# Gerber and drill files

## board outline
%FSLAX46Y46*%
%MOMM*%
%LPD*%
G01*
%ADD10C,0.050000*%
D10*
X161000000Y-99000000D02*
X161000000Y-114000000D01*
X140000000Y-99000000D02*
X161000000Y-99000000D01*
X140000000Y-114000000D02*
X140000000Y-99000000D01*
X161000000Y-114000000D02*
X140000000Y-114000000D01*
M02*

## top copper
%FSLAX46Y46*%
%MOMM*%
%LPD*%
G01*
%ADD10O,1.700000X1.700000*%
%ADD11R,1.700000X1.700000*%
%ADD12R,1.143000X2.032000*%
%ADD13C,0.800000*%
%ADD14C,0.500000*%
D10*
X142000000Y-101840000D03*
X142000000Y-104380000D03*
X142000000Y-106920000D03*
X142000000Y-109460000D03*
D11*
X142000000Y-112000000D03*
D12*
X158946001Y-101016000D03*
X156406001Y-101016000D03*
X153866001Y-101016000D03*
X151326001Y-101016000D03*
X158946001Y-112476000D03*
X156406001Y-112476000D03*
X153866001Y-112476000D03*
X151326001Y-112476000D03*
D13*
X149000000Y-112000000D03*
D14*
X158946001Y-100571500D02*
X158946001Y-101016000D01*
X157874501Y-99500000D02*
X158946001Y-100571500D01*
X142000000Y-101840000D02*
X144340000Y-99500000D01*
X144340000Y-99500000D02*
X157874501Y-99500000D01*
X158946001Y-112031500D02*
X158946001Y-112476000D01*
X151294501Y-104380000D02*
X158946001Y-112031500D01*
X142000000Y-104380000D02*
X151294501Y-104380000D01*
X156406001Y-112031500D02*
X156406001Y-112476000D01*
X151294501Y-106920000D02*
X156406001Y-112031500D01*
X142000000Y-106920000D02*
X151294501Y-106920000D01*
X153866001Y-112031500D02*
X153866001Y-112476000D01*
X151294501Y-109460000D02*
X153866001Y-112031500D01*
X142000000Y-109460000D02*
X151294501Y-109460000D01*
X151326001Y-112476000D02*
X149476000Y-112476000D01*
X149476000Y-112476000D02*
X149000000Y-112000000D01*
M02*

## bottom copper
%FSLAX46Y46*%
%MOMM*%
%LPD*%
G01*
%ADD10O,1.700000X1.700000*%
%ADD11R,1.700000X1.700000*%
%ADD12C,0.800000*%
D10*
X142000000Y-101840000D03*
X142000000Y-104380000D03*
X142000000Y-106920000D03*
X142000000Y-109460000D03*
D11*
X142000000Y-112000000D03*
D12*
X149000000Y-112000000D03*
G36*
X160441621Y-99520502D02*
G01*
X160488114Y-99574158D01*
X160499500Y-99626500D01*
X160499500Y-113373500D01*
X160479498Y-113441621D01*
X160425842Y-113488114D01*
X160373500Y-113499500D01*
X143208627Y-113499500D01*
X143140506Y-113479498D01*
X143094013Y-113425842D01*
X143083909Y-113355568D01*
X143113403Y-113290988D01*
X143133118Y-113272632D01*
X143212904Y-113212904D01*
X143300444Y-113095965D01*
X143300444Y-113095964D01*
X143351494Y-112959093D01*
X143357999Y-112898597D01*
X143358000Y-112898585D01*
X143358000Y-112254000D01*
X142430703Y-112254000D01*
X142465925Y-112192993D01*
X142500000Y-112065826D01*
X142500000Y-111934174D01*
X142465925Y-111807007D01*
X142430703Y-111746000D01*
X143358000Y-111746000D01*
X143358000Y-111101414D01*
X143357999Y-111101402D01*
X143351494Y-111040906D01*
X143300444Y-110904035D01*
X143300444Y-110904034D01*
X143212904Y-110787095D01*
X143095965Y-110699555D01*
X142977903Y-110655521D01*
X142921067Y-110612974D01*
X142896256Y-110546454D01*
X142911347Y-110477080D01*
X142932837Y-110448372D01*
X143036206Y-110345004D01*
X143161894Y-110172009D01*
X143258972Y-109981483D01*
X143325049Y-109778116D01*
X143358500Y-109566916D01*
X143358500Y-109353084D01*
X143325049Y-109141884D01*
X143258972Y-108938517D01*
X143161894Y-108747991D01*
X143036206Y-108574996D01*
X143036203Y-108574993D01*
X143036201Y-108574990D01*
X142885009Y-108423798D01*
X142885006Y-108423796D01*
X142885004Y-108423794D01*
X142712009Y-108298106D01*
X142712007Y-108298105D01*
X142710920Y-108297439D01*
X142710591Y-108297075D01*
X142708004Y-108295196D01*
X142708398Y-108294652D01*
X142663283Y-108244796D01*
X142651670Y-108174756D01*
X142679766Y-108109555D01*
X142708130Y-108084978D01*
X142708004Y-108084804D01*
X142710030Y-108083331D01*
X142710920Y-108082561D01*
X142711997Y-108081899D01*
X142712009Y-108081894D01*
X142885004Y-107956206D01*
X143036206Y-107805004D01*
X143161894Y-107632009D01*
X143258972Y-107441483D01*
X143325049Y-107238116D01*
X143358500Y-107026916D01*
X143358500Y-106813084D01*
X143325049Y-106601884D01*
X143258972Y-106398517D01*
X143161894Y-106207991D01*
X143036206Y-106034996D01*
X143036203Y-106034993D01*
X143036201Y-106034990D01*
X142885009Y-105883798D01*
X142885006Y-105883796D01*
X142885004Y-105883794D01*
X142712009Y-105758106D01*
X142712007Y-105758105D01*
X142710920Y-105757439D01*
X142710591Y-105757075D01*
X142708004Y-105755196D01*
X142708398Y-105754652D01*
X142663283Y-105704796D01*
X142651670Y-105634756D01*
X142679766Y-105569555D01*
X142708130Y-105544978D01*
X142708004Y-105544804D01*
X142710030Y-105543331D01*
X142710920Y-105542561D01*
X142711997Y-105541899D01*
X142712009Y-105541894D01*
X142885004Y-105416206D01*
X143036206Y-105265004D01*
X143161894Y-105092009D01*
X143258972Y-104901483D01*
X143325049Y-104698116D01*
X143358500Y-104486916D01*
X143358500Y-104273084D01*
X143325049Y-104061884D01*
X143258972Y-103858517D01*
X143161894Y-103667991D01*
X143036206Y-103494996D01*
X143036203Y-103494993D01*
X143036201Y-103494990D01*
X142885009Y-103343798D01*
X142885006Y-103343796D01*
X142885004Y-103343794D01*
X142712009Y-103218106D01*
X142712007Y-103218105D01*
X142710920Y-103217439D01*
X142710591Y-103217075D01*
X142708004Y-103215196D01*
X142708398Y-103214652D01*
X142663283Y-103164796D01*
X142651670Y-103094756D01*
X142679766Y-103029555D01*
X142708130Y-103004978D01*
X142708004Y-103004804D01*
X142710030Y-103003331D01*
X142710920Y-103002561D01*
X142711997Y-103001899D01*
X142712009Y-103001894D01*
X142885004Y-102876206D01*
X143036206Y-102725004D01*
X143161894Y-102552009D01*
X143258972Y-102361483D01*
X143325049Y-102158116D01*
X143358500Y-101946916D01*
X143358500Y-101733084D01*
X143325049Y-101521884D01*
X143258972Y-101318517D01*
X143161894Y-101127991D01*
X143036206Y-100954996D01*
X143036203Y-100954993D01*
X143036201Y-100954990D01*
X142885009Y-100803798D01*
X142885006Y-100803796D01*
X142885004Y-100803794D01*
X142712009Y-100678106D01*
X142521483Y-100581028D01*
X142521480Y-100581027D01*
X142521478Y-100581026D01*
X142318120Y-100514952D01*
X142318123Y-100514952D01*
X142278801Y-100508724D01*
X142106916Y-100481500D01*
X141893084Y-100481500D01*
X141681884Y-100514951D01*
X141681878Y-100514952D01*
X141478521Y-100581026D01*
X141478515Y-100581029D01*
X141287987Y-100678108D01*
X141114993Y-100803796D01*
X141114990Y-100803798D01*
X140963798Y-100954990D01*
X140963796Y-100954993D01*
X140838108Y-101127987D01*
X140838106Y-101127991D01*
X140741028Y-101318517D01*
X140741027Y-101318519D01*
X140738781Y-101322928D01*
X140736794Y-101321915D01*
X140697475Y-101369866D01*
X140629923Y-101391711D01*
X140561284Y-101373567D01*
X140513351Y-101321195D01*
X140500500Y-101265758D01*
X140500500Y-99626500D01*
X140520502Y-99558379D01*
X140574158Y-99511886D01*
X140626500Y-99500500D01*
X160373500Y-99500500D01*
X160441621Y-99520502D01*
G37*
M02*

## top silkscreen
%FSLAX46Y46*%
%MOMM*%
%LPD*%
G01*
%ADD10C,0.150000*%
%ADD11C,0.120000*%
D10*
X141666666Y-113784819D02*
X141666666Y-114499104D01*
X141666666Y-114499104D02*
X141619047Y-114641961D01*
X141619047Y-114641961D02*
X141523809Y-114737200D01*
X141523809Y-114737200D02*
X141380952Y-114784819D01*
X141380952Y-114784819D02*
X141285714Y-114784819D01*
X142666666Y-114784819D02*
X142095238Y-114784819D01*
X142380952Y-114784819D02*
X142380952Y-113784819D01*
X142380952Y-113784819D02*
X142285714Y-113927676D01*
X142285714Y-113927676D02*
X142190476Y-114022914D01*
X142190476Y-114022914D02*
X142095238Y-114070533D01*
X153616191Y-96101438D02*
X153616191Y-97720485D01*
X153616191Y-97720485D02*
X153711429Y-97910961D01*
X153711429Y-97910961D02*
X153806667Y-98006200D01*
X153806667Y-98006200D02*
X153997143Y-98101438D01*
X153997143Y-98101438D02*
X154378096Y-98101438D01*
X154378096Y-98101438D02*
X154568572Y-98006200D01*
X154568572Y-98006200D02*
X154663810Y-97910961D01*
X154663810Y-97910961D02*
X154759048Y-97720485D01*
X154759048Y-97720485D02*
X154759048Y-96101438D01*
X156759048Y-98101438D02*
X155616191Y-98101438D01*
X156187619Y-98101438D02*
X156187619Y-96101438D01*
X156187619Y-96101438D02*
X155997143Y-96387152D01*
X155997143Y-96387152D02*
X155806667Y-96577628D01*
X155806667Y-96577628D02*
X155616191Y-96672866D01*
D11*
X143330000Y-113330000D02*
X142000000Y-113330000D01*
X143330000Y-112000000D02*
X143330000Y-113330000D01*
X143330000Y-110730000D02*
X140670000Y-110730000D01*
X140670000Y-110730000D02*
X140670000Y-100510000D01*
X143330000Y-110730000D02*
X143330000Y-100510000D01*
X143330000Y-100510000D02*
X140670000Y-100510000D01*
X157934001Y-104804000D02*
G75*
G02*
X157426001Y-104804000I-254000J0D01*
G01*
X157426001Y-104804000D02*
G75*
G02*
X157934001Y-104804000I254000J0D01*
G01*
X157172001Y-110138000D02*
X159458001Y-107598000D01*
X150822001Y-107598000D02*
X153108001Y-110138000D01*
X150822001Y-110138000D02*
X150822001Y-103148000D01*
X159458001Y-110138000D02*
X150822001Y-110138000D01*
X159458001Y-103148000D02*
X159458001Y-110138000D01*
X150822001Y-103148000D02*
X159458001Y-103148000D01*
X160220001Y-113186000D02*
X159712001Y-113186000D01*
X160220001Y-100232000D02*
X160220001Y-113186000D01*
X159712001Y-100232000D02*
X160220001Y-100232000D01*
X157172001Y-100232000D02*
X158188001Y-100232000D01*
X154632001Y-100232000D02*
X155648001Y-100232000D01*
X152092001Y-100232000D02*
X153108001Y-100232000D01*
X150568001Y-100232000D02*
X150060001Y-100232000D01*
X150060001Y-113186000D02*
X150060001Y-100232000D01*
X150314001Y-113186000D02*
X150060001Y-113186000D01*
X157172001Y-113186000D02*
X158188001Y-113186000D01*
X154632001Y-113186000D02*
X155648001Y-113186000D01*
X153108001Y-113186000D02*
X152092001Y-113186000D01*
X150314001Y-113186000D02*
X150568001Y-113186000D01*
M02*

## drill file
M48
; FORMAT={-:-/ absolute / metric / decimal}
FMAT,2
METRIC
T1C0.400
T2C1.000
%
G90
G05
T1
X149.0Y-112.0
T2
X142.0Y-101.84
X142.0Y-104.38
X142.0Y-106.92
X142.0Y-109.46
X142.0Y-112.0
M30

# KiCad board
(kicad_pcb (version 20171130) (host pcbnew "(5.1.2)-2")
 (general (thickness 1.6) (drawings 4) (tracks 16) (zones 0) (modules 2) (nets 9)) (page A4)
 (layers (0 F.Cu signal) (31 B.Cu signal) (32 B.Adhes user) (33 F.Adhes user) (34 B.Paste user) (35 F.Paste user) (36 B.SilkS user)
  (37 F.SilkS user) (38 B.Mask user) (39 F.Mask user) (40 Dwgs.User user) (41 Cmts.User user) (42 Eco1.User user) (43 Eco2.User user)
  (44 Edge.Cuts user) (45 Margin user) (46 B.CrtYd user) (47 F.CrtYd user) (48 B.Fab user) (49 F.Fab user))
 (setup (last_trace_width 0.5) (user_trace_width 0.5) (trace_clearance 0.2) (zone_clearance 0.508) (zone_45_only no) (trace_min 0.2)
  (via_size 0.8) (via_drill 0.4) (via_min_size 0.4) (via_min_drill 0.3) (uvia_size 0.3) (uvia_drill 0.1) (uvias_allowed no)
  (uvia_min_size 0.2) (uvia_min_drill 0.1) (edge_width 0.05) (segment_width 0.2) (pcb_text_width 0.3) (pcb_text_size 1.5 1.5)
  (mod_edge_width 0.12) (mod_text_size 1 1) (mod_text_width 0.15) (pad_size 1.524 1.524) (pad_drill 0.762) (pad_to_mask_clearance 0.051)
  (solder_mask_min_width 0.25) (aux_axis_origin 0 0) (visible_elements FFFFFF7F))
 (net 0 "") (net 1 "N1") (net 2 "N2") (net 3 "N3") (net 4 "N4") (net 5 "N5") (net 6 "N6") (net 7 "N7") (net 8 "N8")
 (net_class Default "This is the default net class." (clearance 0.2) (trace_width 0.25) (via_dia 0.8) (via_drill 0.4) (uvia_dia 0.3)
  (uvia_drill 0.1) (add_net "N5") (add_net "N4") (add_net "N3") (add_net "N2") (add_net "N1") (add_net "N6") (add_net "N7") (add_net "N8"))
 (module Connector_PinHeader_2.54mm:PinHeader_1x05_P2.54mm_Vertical (layer F.Cu) (at 142 112 180)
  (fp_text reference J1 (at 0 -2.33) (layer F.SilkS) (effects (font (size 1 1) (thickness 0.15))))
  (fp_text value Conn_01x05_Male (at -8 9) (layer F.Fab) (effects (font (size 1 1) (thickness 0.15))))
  (fp_line (start -1.33 -1.33) (end 0 -1.33) (layer F.SilkS) (width 0.12))
  (fp_line (start -1.33 0) (end -1.33 -1.33) (layer F.SilkS) (width 0.12))
  (fp_line (start -1.33 1.27) (end 1.33 1.27) (layer F.SilkS) (width 0.12))
  (fp_line (start 1.33 1.27) (end 1.33 11.49) (layer F.SilkS) (width 0.12))
  (fp_line (start -1.33 1.27) (end -1.33 11.49) (layer F.SilkS) (width 0.12))
  (fp_line (start -1.33 11.49) (end 1.33 11.49) (layer F.SilkS) (width 0.12))
  (pad 5 thru_hole oval (at 0 10.16 180) (size 1.7 1.7) (drill 1) (layers *.Cu *.Mask) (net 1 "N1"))
  (pad 4 thru_hole oval (at 0 7.62 180) (size 1.7 1.7) (drill 1) (layers *.Cu *.Mask) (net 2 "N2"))
  (pad 3 thru_hole oval (at 0 5.08 180) (size 1.7 1.7) (drill 1) (layers *.Cu *.Mask) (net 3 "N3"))
  (pad 2 thru_hole oval (at 0 2.54 180) (size 1.7 1.7) (drill 1) (layers *.Cu *.Mask) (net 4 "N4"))
  (pad 1 thru_hole rect (at 0 0 180) (size 1.7 1.7) (drill 1) (layers *.Cu *.Mask) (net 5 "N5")))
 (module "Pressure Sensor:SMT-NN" (layer F.Cu) (at 155.140001 107.598)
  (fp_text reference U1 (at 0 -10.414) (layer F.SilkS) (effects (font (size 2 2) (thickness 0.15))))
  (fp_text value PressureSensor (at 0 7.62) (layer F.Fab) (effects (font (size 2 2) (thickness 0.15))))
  (fp_circle (center 2.54 -2.794) (end 2.54 -3.048) (layer F.SilkS) (width 0.12))
  (fp_line (start 2.032 2.54) (end 4.318 0) (layer F.SilkS) (width 0.12))
  (fp_line (start -4.318 0) (end -2.032 2.54) (layer F.SilkS) (width 0.12))
  (fp_line (start -4.318 2.54) (end -4.318 -4.45) (layer F.SilkS) (width 0.12))
  (fp_line (start 4.318 2.54) (end -4.318 2.54) (layer F.SilkS) (width 0.12))
  (fp_line (start 4.318 -4.45) (end 4.318 2.54) (layer F.SilkS) (width 0.12))
  (fp_line (start -4.318 -4.45) (end 4.318 -4.45) (layer F.SilkS) (width 0.12))
  (fp_line (start 5.08 5.588) (end 4.572 5.588) (layer F.SilkS) (width 0.12))
  (fp_line (start 5.08 -7.366) (end 5.08 5.588) (layer F.SilkS) (width 0.12))
  (fp_line (start 4.572 -7.366) (end 5.08 -7.366) (layer F.SilkS) (width 0.12))
  (fp_line (start 2.032 -7.366) (end 3.048 -7.366) (layer F.SilkS) (width 0.12))
  (fp_line (start -0.508 -7.366) (end 0.508 -7.366) (layer F.SilkS) (width 0.12))
  (fp_line (start -3.048 -7.366) (end -2.032 -7.366) (layer F.SilkS) (width 0.12))
  (fp_line (start -4.572 -7.366) (end -5.08 -7.366) (layer F.SilkS) (width 0.12))
  (fp_line (start -5.08 5.588) (end -5.08 -7.366) (layer F.SilkS) (width 0.12))
  (fp_line (start -4.826 5.588) (end -5.08 5.588) (layer F.SilkS) (width 0.12))
  (fp_line (start 2.032 5.588) (end 3.048 5.588) (layer F.SilkS) (width 0.12))
  (fp_line (start -0.508 5.588) (end 0.508 5.588) (layer F.SilkS) (width 0.12))
  (fp_line (start -2.032 5.588) (end -3.048 5.588) (layer F.SilkS) (width 0.12))
  (fp_line (start -4.826 5.588) (end -4.572 5.588) (layer F.SilkS) (width 0.12))
  (pad 5 smd rect (at 3.806 -6.582) (size 1.143 2.032) (layers F.Cu F.Paste F.Mask) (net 1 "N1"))
  (pad 6 smd rect (at 1.266 -6.582) (size 1.143 2.032) (layers F.Cu F.Paste F.Mask) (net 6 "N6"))
  (pad 7 smd rect (at -1.274 -6.582) (size 1.143 2.032) (layers F.Cu F.Paste F.Mask) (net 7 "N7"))
  (pad 8 smd rect (at -3.814 -6.582) (size 1.143 2.032) (layers F.Cu F.Paste F.Mask) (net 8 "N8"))
  (pad 4 smd rect (at 3.806 4.878) (size 1.143 2.032) (layers F.Cu F.Paste F.Mask) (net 2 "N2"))
  (pad 3 smd rect (at 1.266 4.878) (size 1.143 2.032) (layers F.Cu F.Paste F.Mask) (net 3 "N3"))
  (pad 2 smd rect (at -1.274 4.878) (size 1.143 2.032) (layers F.Cu F.Paste F.Mask) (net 4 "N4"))
  (pad 1 smd rect (at -3.814 4.878) (size 1.143 2.032) (layers F.Cu F.Paste F.Mask) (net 5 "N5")))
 (gr_line (start 161 99) (end 161 114) (layer Edge.Cuts) (width 0.05))
 (gr_line (start 140 99) (end 161 99) (layer Edge.Cuts) (width 0.05))
 (gr_line (start 140 114) (end 140 99) (layer Edge.Cuts) (width 0.05))
 (gr_line (start 161 114) (end 140 114) (layer Edge.Cuts) (width 0.05))
 (segment (start 158.946001 100.5715) (end 158.946001 101.016) (width 0.5) (layer F.Cu) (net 1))
 (segment (start 157.874501 99.5) (end 158.946001 100.5715) (width 0.5) (layer F.Cu) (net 1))
 (segment (start 142 101.84) (end 144.34 99.5) (width 0.5) (layer F.Cu) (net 1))
 (segment (start 144.34 99.5) (end 157.874501 99.5) (width 0.5) (layer F.Cu) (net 1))
 (segment (start 158.946001 112.0315) (end 158.946001 112.476) (width 0.5) (layer F.Cu) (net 2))
 (segment (start 151.294501 104.38) (end 158.946001 112.0315) (width 0.5) (layer F.Cu) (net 2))
 (segment (start 142 104.38) (end 151.294501 104.38) (width 0.5) (layer F.Cu) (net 2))
 (segment (start 156.406001 112.0315) (end 156.406001 112.476) (width 0.5) (layer F.Cu) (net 3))
 (segment (start 151.294501 106.92) (end 156.406001 112.0315) (width 0.5) (layer F.Cu) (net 3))
 (segment (start 142 106.92) (end 151.294501 106.92) (width 0.5) (layer F.Cu) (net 3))
 (segment (start 153.866001 112.0315) (end 153.866001 112.476) (width 0.5) (layer F.Cu) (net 4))
 (segment (start 151.294501 109.46) (end 153.866001 112.0315) (width 0.5) (layer F.Cu) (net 4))
 (segment (start 142 109.46) (end 151.294501 109.46) (width 0.5) (layer F.Cu) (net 4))
 (via (at 149 112) (size 0.8) (drill 0.4) (layers F.Cu B.Cu) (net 5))
 (segment (start 151.326001 112.476) (end 149.476 112.476) (width 0.5) (layer F.Cu) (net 5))
 (segment (start 149.476 112.476) (end 149 112) (width 0.5) (layer F.Cu) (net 5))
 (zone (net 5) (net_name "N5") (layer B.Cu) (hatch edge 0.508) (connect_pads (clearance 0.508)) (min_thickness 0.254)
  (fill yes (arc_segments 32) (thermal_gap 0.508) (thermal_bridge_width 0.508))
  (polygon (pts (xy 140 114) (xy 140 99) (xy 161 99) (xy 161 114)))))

